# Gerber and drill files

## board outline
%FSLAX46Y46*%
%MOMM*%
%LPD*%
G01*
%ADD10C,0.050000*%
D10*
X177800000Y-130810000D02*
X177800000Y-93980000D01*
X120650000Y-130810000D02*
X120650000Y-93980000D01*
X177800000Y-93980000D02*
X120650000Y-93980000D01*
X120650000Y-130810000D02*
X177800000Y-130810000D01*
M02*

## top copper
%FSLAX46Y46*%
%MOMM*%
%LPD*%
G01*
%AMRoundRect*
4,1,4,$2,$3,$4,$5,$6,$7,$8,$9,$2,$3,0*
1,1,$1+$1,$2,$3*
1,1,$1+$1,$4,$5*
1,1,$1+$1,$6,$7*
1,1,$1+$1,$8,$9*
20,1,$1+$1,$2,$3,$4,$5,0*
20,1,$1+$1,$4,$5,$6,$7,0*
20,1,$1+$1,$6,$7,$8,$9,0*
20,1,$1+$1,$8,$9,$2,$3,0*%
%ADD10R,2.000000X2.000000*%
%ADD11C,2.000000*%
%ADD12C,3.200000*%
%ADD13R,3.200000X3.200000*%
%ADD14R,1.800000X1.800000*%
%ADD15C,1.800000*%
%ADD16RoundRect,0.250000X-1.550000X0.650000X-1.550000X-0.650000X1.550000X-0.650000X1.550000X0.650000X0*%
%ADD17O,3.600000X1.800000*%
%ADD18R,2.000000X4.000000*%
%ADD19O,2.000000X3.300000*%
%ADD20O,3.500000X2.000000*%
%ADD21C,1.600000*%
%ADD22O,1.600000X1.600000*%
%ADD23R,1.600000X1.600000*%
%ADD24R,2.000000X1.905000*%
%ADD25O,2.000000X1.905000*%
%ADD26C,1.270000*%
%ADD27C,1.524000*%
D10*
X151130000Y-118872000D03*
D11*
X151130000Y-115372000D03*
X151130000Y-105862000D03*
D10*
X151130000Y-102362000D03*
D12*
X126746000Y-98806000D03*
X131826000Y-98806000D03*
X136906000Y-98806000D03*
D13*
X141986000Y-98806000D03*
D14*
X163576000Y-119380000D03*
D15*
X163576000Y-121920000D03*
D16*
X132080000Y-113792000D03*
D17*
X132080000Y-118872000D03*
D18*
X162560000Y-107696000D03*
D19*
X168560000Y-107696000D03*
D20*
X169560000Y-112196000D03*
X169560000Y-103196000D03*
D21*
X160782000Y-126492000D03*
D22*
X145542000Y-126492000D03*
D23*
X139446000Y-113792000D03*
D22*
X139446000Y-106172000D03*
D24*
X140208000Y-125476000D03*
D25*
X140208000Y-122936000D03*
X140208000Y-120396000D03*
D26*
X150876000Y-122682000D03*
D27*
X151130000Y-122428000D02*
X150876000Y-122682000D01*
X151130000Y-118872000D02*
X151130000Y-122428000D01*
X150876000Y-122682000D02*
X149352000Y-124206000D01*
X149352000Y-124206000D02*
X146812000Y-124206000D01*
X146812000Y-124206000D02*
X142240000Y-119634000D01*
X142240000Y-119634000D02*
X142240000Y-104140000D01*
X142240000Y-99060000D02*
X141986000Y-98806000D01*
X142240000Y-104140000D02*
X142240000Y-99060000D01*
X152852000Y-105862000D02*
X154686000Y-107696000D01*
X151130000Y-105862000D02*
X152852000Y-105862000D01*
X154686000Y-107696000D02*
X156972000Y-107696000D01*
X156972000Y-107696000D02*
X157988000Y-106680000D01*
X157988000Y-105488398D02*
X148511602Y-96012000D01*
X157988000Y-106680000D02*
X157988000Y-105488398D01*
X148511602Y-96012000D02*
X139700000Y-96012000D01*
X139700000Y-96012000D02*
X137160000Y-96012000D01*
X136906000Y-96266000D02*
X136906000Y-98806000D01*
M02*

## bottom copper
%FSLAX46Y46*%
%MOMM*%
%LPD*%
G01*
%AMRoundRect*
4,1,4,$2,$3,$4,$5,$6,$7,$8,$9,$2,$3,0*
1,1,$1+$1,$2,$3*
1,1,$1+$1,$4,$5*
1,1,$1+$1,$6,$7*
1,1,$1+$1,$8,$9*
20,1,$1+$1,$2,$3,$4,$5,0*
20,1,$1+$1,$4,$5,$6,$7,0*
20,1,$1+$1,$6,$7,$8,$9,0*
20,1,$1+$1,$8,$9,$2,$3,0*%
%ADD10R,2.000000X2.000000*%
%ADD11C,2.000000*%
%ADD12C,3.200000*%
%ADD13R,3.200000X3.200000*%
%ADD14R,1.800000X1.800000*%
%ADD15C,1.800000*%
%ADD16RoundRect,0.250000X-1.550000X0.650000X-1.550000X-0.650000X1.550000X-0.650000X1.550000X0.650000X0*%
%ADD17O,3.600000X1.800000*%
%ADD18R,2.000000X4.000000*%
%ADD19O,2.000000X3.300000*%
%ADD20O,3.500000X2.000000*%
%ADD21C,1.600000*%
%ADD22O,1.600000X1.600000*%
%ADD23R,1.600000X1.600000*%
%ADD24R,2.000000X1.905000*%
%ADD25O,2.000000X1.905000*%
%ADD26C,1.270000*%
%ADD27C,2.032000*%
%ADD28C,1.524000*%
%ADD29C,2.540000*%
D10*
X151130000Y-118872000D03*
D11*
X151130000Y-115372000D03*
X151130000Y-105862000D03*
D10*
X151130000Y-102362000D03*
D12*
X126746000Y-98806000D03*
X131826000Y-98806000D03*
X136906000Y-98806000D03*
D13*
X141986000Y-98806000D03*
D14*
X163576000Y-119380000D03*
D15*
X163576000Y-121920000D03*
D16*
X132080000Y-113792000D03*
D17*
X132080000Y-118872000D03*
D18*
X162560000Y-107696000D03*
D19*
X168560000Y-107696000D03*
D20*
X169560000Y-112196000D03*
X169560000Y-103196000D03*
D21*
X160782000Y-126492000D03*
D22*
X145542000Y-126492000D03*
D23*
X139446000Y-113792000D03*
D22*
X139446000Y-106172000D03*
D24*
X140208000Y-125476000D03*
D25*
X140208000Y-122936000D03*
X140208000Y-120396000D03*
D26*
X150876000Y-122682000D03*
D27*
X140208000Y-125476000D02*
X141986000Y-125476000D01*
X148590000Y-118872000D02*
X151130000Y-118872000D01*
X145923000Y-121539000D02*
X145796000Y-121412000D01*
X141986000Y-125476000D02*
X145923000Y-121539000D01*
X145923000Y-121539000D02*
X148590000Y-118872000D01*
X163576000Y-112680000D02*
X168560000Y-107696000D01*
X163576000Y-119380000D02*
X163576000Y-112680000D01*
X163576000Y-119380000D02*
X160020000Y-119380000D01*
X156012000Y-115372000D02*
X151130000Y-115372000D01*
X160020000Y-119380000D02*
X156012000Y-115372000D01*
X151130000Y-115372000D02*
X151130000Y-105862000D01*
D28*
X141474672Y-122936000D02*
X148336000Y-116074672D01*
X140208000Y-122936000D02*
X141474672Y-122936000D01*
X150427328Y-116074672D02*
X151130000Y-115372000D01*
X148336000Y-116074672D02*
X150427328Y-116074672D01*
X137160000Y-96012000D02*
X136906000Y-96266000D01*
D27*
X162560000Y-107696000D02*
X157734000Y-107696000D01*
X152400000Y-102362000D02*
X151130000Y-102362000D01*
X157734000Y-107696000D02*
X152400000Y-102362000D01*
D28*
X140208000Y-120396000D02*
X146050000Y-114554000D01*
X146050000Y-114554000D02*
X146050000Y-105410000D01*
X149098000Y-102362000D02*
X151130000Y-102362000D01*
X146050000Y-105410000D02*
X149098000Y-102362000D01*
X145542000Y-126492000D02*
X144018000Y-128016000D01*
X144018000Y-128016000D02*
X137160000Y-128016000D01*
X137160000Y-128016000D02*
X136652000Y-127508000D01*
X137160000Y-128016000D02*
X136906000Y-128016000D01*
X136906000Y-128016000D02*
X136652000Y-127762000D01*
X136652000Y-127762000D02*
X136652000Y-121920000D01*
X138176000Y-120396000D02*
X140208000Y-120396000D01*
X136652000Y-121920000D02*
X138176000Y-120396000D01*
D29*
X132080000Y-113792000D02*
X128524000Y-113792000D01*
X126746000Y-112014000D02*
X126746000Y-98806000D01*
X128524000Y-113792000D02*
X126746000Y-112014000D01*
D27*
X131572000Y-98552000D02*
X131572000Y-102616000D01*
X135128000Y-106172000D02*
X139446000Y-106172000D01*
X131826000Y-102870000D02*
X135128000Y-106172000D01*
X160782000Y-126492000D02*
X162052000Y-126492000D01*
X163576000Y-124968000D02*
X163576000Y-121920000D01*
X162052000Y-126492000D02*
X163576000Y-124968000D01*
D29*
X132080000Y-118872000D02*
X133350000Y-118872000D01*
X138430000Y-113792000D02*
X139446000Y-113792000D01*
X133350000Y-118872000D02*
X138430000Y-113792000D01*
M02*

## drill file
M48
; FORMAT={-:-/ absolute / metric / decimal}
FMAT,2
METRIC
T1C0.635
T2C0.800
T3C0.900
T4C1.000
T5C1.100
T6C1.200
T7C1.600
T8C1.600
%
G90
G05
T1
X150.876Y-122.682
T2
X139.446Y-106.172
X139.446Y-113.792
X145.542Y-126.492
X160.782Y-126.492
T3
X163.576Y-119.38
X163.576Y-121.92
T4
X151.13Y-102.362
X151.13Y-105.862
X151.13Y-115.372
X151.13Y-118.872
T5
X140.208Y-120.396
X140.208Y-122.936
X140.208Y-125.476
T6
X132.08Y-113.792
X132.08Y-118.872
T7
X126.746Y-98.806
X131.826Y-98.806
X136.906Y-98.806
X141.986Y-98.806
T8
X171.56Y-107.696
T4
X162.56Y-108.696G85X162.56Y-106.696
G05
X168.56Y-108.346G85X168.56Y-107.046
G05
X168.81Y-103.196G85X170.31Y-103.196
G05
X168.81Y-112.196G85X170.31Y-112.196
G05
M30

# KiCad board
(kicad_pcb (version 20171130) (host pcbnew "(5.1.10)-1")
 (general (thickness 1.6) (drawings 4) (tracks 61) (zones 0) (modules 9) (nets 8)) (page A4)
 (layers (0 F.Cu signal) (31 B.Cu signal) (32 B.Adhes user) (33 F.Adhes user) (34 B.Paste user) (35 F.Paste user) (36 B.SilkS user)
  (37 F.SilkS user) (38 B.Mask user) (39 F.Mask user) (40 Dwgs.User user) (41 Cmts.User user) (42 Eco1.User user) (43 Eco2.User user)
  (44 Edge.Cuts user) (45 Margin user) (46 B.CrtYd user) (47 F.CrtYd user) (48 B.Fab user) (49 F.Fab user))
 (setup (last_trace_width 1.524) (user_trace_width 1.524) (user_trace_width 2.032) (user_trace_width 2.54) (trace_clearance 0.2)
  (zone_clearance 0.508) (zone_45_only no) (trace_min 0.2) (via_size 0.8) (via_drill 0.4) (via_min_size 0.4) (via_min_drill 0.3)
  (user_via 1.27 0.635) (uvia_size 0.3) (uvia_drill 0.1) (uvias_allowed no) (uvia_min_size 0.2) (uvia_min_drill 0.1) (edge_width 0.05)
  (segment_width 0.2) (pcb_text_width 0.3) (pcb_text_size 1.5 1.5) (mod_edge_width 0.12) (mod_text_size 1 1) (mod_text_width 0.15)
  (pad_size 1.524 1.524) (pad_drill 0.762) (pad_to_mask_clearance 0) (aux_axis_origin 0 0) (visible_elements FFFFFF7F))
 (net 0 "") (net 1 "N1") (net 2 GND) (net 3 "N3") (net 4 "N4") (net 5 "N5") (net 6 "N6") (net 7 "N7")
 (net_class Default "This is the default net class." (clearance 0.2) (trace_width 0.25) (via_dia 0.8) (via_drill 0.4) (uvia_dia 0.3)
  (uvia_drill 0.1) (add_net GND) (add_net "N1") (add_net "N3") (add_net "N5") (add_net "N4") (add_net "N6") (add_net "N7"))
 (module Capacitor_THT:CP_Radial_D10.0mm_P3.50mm (layer F.Cu) (at 151.13 118.872 90)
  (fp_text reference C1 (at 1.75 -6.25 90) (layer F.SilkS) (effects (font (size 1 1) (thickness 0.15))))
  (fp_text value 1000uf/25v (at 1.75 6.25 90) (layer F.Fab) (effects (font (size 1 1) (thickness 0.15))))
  (pad 1 thru_hole rect (at 0 0 90) (size 2 2) (drill 1) (layers *.Cu *.Mask) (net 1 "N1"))
  (pad 2 thru_hole circle (at 3.5 0 90) (size 2 2) (drill 1) (layers *.Cu *.Mask) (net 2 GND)))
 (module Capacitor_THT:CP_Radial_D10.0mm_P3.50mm (layer F.Cu) (at 151.13 102.362 270)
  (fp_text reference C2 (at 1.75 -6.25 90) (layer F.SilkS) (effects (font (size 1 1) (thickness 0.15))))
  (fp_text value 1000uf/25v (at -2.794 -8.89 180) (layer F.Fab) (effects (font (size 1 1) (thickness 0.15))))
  (pad 2 thru_hole circle (at 3.5 0 270) (size 2 2) (drill 1) (layers *.Cu *.Mask) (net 2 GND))
  (pad 1 thru_hole rect (at 0 0 270) (size 2 2) (drill 1) (layers *.Cu *.Mask) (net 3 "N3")))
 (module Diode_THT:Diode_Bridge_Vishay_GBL (layer F.Cu) (at 141.986 98.806 180)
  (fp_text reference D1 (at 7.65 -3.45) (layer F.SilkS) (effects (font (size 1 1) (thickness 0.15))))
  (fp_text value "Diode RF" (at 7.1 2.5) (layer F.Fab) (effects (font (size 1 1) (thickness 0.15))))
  (pad 4 thru_hole circle (at 15.24 0) (size 3.2 3.2) (drill 1.6) (layers *.Cu *.Mask) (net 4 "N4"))
  (pad 3 thru_hole circle (at 10.16 0) (size 3.2 3.2) (drill 1.6) (layers *.Cu *.Mask) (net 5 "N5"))
  (pad 2 thru_hole circle (at 5.08 0) (size 3.2 3.2) (drill 1.6) (layers *.Cu *.Mask) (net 2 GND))
  (pad 1 thru_hole rect (at 0 0) (size 3.2 3.2) (drill 1.6) (layers *.Cu *.Mask) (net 1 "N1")))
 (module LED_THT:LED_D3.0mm (layer F.Cu) (at 163.576 119.38 270)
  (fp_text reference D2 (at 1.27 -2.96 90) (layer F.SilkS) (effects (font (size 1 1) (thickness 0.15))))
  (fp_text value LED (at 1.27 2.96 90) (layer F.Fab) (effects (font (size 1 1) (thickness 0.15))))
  (pad 1 thru_hole rect (at 0 0 270) (size 1.8 1.8) (drill 0.9) (layers *.Cu *.Mask) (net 2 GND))
  (pad 2 thru_hole circle (at 2.54 0 270) (size 1.8 1.8) (drill 0.9) (layers *.Cu *.Mask) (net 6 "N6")))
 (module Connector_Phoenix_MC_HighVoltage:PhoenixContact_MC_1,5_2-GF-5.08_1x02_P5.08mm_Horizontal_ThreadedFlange (layer F.Cu)
  (at 132.08 113.792 270)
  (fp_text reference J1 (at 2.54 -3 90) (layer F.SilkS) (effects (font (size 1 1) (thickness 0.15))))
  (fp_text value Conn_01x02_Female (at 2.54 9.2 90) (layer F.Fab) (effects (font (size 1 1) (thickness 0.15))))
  (pad 1 thru_hole roundrect (at 0 0 270) (size 1.8 3.6) (drill 1.2) (layers *.Cu *.Mask) (roundrect_rratio 0.138889) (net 4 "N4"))
  (pad 2 thru_hole oval (at 5.08 0 270) (size 1.8 3.6) (drill 1.2) (layers *.Cu *.Mask) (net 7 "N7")))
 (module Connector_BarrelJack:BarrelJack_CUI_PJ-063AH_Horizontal (layer F.Cu) (at 162.56 107.696 90)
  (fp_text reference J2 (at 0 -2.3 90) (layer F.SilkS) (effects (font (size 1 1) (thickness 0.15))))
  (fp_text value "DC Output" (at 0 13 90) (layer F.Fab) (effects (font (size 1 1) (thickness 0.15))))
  (pad 1 thru_hole rect (at 0 0 90) (size 4 2) (drill oval 3 1) (layers *.Cu *.Mask) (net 2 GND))
  (pad 2 thru_hole oval (at 0 6 90) (size 3.3 2) (drill oval 2.3 1) (layers *.Cu *.Mask) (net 2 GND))
  (pad MP thru_hole oval (at -4.5 7 90) (size 2 3.5) (drill oval 1 2.5) (layers *.Cu *.Mask))
  (pad MP thru_hole oval (at 4.5 7 90) (size 2 3.5) (drill oval 1 2.5) (layers *.Cu *.Mask))
  (pad "" np_thru_hole circle (at 0 9 90) (size 1.6 1.6) (drill 1.6) (layers *.Cu *.Mask)))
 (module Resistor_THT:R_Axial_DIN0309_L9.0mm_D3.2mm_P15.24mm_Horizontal (layer F.Cu) (at 160.782 126.492 180)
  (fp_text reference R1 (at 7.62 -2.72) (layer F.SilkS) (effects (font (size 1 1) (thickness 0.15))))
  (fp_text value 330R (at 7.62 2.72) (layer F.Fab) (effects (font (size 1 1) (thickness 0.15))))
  (pad 1 thru_hole circle (at 0 0 180) (size 1.6 1.6) (drill 0.8) (layers *.Cu *.Mask) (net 6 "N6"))
  (pad 2 thru_hole oval (at 15.24 0 180) (size 1.6 1.6) (drill 0.8) (layers *.Cu *.Mask) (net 3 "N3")))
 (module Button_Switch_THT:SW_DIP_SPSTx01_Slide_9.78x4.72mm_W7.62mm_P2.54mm (layer F.Cu) (at 139.446 113.792 90)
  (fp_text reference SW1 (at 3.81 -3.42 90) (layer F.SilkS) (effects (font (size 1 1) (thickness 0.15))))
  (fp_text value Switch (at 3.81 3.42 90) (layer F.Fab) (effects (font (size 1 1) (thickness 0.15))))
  (pad 1 thru_hole rect (at 0 0 90) (size 1.6 1.6) (drill 0.8) (layers *.Cu *.Mask) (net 7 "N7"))
  (pad 2 thru_hole oval (at 7.62 0 90) (size 1.6 1.6) (drill 0.8) (layers *.Cu *.Mask) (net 5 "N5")))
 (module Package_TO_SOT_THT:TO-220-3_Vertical (layer F.Cu) (at 140.208 125.476 90)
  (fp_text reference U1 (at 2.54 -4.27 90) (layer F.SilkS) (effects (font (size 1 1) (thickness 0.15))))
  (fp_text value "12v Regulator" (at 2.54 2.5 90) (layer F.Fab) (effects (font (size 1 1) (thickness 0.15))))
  (pad 1 thru_hole rect (at 0 0 90) (size 1.905 2) (drill 1.1) (layers *.Cu *.Mask) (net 1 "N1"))
  (pad 2 thru_hole oval (at 2.54 0 90) (size 1.905 2) (drill 1.1) (layers *.Cu *.Mask) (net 2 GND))
  (pad 3 thru_hole oval (at 5.08 0 90) (size 1.905 2) (drill 1.1) (layers *.Cu *.Mask) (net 3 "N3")))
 (gr_line (start 177.8 130.81) (end 177.8 93.98) (layer Edge.Cuts) (width 0.05))
 (gr_line (start 120.65 130.81) (end 120.65 93.98) (layer Edge.Cuts) (width 0.05))
 (gr_line (start 177.8 93.98) (end 120.65 93.98) (layer Edge.Cuts) (width 0.05))
 (gr_line (start 120.65 130.81) (end 177.8 130.81) (layer Edge.Cuts) (width 0.05))
 (segment (start 140.208 125.476) (end 141.986 125.476) (width 2.032) (layer B.Cu) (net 1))
 (segment (start 148.59 118.872) (end 151.13 118.872) (width 2.032) (layer B.Cu) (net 1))
 (segment (start 145.923 121.539) (end 145.796 121.412) (width 2.032) (layer B.Cu) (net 1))
 (segment (start 141.986 125.476) (end 145.923 121.539) (width 2.032) (layer B.Cu) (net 1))
 (segment (start 145.923 121.539) (end 148.59 118.872) (width 2.032) (layer B.Cu) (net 1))
 (via (at 150.876 122.682) (size 1.27) (drill 0.635) (layers F.Cu B.Cu) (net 1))
 (segment (start 151.13 122.428) (end 150.876 122.682) (width 1.524) (layer F.Cu) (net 1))
 (segment (start 151.13 118.872) (end 151.13 122.428) (width 1.524) (layer F.Cu) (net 1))
 (segment (start 150.876 122.682) (end 149.352 124.206) (width 1.524) (layer F.Cu) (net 1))
 (segment (start 149.352 124.206) (end 146.812 124.206) (width 1.524) (layer F.Cu) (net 1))
 (segment (start 146.812 124.206) (end 142.24 119.634) (width 1.524) (layer F.Cu) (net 1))
 (segment (start 142.24 119.634) (end 142.24 104.14) (width 1.524) (layer F.Cu) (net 1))
 (segment (start 142.24 99.06) (end 141.986 98.806) (width 1.524) (layer F.Cu) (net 1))
 (segment (start 142.24 104.14) (end 142.24 99.06) (width 1.524) (layer F.Cu) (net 1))
 (segment (start 163.576 112.68) (end 168.56 107.696) (width 2.032) (layer B.Cu) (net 2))
 (segment (start 163.576 119.38) (end 163.576 112.68) (width 2.032) (layer B.Cu) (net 2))
 (segment (start 163.576 119.38) (end 160.02 119.38) (width 2.032) (layer B.Cu) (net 2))
 (segment (start 156.012 115.372) (end 151.13 115.372) (width 2.032) (layer B.Cu) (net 2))
 (segment (start 160.02 119.38) (end 156.012 115.372) (width 2.032) (layer B.Cu) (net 2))
 (segment (start 151.13 115.372) (end 151.13 105.862) (width 2.032) (layer B.Cu) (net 2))
 (segment (start 141.474672 122.936) (end 148.336 116.074672) (width 1.524) (layer B.Cu) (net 2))
 (segment (start 140.208 122.936) (end 141.474672 122.936) (width 1.524) (layer B.Cu) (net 2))
 (segment (start 150.427328 116.074672) (end 151.13 115.372) (width 1.524) (layer B.Cu) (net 2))
 (segment (start 148.336 116.074672) (end 150.427328 116.074672) (width 1.524) (layer B.Cu) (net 2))
 (segment (start 152.852 105.862) (end 154.686 107.696) (width 1.524) (layer F.Cu) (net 2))
 (segment (start 151.13 105.862) (end 152.852 105.862) (width 1.524) (layer F.Cu) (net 2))
 (segment (start 154.686 107.696) (end 156.972 107.696) (width 1.524) (layer F.Cu) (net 2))
 (segment (start 156.972 107.696) (end 157.988 106.68) (width 1.524) (layer F.Cu) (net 2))
 (segment (start 157.988 105.488398) (end 148.511602 96.012) (width 1.524) (layer F.Cu) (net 2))
 (segment (start 157.988 106.68) (end 157.988 105.488398) (width 1.524) (layer F.Cu) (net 2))
 (segment (start 148.511602 96.012) (end 139.7 96.012) (width 1.524) (layer F.Cu) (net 2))
 (segment (start 139.7 96.012) (end 137.16 96.012) (width 1.524) (layer F.Cu) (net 2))
 (segment (start 136.906 96.266) (end 136.906 98.806) (width 1.524) (layer F.Cu) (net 2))
 (segment (start 137.16 96.012) (end 136.906 96.266) (width 1.524) (layer B.Cu) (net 2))
 (segment (start 162.56 107.696) (end 157.734 107.696) (width 2.032) (layer B.Cu) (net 2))
 (segment (start 152.4 102.362) (end 151.13 102.362) (width 2.032) (layer B.Cu) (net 3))
 (segment (start 157.734 107.696) (end 152.4 102.362) (width 2.032) (layer B.Cu) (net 2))
 (segment (start 140.208 120.396) (end 146.05 114.554) (width 1.524) (layer B.Cu) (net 3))
 (segment (start 146.05 114.554) (end 146.05 105.41) (width 1.524) (layer B.Cu) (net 3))
 (segment (start 149.098 102.362) (end 151.13 102.362) (width 1.524) (layer B.Cu) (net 3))
 (segment (start 146.05 105.41) (end 149.098 102.362) (width 1.524) (layer B.Cu) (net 3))
 (segment (start 145.542 126.492) (end 144.018 128.016) (width 1.524) (layer B.Cu) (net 3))
 (segment (start 144.018 128.016) (end 137.16 128.016) (width 1.524) (layer B.Cu) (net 3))
 (segment (start 137.16 128.016) (end 136.652 127.508) (width 1.524) (layer B.Cu) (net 3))
 (segment (start 137.16 128.016) (end 136.906 128.016) (width 1.524) (layer B.Cu) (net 3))
 (segment (start 136.906 128.016) (end 136.652 127.762) (width 1.524) (layer B.Cu) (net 3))
 (segment (start 136.652 127.762) (end 136.652 121.92) (width 1.524) (layer B.Cu) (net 3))
 (segment (start 138.176 120.396) (end 140.208 120.396) (width 1.524) (layer B.Cu) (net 3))
 (segment (start 136.652 121.92) (end 138.176 120.396) (width 1.524) (layer B.Cu) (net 3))
 (segment (start 132.08 113.792) (end 128.524 113.792) (width 2.54) (layer B.Cu) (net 4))
 (segment (start 126.746 112.014) (end 126.746 98.806) (width 2.54) (layer B.Cu) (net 4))
 (segment (start 128.524 113.792) (end 126.746 112.014) (width 2.54) (layer B.Cu) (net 4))
 (segment (start 131.572 98.552) (end 131.572 102.616) (width 2.032) (layer B.Cu) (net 5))
 (segment (start 135.128 106.172) (end 139.446 106.172) (width 2.032) (layer B.Cu) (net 5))
 (segment (start 131.826 102.87) (end 135.128 106.172) (width 2.032) (layer B.Cu) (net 5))
 (segment (start 160.782 126.492) (end 162.052 126.492) (width 2.032) (layer B.Cu) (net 6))
 (segment (start 163.576 124.968) (end 163.576 121.92) (width 2.032) (layer B.Cu) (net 6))
 (segment (start 162.052 126.492) (end 163.576 124.968) (width 2.032) (layer B.Cu) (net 6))
 (segment (start 132.08 118.872) (end 133.35 118.872) (width 2.54) (layer B.Cu) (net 7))
 (segment (start 138.43 113.792) (end 139.446 113.792) (width 2.54) (layer B.Cu) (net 7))
 (segment (start 133.35 118.872) (end 138.43 113.792) (width 2.54) (layer B.Cu) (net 7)))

